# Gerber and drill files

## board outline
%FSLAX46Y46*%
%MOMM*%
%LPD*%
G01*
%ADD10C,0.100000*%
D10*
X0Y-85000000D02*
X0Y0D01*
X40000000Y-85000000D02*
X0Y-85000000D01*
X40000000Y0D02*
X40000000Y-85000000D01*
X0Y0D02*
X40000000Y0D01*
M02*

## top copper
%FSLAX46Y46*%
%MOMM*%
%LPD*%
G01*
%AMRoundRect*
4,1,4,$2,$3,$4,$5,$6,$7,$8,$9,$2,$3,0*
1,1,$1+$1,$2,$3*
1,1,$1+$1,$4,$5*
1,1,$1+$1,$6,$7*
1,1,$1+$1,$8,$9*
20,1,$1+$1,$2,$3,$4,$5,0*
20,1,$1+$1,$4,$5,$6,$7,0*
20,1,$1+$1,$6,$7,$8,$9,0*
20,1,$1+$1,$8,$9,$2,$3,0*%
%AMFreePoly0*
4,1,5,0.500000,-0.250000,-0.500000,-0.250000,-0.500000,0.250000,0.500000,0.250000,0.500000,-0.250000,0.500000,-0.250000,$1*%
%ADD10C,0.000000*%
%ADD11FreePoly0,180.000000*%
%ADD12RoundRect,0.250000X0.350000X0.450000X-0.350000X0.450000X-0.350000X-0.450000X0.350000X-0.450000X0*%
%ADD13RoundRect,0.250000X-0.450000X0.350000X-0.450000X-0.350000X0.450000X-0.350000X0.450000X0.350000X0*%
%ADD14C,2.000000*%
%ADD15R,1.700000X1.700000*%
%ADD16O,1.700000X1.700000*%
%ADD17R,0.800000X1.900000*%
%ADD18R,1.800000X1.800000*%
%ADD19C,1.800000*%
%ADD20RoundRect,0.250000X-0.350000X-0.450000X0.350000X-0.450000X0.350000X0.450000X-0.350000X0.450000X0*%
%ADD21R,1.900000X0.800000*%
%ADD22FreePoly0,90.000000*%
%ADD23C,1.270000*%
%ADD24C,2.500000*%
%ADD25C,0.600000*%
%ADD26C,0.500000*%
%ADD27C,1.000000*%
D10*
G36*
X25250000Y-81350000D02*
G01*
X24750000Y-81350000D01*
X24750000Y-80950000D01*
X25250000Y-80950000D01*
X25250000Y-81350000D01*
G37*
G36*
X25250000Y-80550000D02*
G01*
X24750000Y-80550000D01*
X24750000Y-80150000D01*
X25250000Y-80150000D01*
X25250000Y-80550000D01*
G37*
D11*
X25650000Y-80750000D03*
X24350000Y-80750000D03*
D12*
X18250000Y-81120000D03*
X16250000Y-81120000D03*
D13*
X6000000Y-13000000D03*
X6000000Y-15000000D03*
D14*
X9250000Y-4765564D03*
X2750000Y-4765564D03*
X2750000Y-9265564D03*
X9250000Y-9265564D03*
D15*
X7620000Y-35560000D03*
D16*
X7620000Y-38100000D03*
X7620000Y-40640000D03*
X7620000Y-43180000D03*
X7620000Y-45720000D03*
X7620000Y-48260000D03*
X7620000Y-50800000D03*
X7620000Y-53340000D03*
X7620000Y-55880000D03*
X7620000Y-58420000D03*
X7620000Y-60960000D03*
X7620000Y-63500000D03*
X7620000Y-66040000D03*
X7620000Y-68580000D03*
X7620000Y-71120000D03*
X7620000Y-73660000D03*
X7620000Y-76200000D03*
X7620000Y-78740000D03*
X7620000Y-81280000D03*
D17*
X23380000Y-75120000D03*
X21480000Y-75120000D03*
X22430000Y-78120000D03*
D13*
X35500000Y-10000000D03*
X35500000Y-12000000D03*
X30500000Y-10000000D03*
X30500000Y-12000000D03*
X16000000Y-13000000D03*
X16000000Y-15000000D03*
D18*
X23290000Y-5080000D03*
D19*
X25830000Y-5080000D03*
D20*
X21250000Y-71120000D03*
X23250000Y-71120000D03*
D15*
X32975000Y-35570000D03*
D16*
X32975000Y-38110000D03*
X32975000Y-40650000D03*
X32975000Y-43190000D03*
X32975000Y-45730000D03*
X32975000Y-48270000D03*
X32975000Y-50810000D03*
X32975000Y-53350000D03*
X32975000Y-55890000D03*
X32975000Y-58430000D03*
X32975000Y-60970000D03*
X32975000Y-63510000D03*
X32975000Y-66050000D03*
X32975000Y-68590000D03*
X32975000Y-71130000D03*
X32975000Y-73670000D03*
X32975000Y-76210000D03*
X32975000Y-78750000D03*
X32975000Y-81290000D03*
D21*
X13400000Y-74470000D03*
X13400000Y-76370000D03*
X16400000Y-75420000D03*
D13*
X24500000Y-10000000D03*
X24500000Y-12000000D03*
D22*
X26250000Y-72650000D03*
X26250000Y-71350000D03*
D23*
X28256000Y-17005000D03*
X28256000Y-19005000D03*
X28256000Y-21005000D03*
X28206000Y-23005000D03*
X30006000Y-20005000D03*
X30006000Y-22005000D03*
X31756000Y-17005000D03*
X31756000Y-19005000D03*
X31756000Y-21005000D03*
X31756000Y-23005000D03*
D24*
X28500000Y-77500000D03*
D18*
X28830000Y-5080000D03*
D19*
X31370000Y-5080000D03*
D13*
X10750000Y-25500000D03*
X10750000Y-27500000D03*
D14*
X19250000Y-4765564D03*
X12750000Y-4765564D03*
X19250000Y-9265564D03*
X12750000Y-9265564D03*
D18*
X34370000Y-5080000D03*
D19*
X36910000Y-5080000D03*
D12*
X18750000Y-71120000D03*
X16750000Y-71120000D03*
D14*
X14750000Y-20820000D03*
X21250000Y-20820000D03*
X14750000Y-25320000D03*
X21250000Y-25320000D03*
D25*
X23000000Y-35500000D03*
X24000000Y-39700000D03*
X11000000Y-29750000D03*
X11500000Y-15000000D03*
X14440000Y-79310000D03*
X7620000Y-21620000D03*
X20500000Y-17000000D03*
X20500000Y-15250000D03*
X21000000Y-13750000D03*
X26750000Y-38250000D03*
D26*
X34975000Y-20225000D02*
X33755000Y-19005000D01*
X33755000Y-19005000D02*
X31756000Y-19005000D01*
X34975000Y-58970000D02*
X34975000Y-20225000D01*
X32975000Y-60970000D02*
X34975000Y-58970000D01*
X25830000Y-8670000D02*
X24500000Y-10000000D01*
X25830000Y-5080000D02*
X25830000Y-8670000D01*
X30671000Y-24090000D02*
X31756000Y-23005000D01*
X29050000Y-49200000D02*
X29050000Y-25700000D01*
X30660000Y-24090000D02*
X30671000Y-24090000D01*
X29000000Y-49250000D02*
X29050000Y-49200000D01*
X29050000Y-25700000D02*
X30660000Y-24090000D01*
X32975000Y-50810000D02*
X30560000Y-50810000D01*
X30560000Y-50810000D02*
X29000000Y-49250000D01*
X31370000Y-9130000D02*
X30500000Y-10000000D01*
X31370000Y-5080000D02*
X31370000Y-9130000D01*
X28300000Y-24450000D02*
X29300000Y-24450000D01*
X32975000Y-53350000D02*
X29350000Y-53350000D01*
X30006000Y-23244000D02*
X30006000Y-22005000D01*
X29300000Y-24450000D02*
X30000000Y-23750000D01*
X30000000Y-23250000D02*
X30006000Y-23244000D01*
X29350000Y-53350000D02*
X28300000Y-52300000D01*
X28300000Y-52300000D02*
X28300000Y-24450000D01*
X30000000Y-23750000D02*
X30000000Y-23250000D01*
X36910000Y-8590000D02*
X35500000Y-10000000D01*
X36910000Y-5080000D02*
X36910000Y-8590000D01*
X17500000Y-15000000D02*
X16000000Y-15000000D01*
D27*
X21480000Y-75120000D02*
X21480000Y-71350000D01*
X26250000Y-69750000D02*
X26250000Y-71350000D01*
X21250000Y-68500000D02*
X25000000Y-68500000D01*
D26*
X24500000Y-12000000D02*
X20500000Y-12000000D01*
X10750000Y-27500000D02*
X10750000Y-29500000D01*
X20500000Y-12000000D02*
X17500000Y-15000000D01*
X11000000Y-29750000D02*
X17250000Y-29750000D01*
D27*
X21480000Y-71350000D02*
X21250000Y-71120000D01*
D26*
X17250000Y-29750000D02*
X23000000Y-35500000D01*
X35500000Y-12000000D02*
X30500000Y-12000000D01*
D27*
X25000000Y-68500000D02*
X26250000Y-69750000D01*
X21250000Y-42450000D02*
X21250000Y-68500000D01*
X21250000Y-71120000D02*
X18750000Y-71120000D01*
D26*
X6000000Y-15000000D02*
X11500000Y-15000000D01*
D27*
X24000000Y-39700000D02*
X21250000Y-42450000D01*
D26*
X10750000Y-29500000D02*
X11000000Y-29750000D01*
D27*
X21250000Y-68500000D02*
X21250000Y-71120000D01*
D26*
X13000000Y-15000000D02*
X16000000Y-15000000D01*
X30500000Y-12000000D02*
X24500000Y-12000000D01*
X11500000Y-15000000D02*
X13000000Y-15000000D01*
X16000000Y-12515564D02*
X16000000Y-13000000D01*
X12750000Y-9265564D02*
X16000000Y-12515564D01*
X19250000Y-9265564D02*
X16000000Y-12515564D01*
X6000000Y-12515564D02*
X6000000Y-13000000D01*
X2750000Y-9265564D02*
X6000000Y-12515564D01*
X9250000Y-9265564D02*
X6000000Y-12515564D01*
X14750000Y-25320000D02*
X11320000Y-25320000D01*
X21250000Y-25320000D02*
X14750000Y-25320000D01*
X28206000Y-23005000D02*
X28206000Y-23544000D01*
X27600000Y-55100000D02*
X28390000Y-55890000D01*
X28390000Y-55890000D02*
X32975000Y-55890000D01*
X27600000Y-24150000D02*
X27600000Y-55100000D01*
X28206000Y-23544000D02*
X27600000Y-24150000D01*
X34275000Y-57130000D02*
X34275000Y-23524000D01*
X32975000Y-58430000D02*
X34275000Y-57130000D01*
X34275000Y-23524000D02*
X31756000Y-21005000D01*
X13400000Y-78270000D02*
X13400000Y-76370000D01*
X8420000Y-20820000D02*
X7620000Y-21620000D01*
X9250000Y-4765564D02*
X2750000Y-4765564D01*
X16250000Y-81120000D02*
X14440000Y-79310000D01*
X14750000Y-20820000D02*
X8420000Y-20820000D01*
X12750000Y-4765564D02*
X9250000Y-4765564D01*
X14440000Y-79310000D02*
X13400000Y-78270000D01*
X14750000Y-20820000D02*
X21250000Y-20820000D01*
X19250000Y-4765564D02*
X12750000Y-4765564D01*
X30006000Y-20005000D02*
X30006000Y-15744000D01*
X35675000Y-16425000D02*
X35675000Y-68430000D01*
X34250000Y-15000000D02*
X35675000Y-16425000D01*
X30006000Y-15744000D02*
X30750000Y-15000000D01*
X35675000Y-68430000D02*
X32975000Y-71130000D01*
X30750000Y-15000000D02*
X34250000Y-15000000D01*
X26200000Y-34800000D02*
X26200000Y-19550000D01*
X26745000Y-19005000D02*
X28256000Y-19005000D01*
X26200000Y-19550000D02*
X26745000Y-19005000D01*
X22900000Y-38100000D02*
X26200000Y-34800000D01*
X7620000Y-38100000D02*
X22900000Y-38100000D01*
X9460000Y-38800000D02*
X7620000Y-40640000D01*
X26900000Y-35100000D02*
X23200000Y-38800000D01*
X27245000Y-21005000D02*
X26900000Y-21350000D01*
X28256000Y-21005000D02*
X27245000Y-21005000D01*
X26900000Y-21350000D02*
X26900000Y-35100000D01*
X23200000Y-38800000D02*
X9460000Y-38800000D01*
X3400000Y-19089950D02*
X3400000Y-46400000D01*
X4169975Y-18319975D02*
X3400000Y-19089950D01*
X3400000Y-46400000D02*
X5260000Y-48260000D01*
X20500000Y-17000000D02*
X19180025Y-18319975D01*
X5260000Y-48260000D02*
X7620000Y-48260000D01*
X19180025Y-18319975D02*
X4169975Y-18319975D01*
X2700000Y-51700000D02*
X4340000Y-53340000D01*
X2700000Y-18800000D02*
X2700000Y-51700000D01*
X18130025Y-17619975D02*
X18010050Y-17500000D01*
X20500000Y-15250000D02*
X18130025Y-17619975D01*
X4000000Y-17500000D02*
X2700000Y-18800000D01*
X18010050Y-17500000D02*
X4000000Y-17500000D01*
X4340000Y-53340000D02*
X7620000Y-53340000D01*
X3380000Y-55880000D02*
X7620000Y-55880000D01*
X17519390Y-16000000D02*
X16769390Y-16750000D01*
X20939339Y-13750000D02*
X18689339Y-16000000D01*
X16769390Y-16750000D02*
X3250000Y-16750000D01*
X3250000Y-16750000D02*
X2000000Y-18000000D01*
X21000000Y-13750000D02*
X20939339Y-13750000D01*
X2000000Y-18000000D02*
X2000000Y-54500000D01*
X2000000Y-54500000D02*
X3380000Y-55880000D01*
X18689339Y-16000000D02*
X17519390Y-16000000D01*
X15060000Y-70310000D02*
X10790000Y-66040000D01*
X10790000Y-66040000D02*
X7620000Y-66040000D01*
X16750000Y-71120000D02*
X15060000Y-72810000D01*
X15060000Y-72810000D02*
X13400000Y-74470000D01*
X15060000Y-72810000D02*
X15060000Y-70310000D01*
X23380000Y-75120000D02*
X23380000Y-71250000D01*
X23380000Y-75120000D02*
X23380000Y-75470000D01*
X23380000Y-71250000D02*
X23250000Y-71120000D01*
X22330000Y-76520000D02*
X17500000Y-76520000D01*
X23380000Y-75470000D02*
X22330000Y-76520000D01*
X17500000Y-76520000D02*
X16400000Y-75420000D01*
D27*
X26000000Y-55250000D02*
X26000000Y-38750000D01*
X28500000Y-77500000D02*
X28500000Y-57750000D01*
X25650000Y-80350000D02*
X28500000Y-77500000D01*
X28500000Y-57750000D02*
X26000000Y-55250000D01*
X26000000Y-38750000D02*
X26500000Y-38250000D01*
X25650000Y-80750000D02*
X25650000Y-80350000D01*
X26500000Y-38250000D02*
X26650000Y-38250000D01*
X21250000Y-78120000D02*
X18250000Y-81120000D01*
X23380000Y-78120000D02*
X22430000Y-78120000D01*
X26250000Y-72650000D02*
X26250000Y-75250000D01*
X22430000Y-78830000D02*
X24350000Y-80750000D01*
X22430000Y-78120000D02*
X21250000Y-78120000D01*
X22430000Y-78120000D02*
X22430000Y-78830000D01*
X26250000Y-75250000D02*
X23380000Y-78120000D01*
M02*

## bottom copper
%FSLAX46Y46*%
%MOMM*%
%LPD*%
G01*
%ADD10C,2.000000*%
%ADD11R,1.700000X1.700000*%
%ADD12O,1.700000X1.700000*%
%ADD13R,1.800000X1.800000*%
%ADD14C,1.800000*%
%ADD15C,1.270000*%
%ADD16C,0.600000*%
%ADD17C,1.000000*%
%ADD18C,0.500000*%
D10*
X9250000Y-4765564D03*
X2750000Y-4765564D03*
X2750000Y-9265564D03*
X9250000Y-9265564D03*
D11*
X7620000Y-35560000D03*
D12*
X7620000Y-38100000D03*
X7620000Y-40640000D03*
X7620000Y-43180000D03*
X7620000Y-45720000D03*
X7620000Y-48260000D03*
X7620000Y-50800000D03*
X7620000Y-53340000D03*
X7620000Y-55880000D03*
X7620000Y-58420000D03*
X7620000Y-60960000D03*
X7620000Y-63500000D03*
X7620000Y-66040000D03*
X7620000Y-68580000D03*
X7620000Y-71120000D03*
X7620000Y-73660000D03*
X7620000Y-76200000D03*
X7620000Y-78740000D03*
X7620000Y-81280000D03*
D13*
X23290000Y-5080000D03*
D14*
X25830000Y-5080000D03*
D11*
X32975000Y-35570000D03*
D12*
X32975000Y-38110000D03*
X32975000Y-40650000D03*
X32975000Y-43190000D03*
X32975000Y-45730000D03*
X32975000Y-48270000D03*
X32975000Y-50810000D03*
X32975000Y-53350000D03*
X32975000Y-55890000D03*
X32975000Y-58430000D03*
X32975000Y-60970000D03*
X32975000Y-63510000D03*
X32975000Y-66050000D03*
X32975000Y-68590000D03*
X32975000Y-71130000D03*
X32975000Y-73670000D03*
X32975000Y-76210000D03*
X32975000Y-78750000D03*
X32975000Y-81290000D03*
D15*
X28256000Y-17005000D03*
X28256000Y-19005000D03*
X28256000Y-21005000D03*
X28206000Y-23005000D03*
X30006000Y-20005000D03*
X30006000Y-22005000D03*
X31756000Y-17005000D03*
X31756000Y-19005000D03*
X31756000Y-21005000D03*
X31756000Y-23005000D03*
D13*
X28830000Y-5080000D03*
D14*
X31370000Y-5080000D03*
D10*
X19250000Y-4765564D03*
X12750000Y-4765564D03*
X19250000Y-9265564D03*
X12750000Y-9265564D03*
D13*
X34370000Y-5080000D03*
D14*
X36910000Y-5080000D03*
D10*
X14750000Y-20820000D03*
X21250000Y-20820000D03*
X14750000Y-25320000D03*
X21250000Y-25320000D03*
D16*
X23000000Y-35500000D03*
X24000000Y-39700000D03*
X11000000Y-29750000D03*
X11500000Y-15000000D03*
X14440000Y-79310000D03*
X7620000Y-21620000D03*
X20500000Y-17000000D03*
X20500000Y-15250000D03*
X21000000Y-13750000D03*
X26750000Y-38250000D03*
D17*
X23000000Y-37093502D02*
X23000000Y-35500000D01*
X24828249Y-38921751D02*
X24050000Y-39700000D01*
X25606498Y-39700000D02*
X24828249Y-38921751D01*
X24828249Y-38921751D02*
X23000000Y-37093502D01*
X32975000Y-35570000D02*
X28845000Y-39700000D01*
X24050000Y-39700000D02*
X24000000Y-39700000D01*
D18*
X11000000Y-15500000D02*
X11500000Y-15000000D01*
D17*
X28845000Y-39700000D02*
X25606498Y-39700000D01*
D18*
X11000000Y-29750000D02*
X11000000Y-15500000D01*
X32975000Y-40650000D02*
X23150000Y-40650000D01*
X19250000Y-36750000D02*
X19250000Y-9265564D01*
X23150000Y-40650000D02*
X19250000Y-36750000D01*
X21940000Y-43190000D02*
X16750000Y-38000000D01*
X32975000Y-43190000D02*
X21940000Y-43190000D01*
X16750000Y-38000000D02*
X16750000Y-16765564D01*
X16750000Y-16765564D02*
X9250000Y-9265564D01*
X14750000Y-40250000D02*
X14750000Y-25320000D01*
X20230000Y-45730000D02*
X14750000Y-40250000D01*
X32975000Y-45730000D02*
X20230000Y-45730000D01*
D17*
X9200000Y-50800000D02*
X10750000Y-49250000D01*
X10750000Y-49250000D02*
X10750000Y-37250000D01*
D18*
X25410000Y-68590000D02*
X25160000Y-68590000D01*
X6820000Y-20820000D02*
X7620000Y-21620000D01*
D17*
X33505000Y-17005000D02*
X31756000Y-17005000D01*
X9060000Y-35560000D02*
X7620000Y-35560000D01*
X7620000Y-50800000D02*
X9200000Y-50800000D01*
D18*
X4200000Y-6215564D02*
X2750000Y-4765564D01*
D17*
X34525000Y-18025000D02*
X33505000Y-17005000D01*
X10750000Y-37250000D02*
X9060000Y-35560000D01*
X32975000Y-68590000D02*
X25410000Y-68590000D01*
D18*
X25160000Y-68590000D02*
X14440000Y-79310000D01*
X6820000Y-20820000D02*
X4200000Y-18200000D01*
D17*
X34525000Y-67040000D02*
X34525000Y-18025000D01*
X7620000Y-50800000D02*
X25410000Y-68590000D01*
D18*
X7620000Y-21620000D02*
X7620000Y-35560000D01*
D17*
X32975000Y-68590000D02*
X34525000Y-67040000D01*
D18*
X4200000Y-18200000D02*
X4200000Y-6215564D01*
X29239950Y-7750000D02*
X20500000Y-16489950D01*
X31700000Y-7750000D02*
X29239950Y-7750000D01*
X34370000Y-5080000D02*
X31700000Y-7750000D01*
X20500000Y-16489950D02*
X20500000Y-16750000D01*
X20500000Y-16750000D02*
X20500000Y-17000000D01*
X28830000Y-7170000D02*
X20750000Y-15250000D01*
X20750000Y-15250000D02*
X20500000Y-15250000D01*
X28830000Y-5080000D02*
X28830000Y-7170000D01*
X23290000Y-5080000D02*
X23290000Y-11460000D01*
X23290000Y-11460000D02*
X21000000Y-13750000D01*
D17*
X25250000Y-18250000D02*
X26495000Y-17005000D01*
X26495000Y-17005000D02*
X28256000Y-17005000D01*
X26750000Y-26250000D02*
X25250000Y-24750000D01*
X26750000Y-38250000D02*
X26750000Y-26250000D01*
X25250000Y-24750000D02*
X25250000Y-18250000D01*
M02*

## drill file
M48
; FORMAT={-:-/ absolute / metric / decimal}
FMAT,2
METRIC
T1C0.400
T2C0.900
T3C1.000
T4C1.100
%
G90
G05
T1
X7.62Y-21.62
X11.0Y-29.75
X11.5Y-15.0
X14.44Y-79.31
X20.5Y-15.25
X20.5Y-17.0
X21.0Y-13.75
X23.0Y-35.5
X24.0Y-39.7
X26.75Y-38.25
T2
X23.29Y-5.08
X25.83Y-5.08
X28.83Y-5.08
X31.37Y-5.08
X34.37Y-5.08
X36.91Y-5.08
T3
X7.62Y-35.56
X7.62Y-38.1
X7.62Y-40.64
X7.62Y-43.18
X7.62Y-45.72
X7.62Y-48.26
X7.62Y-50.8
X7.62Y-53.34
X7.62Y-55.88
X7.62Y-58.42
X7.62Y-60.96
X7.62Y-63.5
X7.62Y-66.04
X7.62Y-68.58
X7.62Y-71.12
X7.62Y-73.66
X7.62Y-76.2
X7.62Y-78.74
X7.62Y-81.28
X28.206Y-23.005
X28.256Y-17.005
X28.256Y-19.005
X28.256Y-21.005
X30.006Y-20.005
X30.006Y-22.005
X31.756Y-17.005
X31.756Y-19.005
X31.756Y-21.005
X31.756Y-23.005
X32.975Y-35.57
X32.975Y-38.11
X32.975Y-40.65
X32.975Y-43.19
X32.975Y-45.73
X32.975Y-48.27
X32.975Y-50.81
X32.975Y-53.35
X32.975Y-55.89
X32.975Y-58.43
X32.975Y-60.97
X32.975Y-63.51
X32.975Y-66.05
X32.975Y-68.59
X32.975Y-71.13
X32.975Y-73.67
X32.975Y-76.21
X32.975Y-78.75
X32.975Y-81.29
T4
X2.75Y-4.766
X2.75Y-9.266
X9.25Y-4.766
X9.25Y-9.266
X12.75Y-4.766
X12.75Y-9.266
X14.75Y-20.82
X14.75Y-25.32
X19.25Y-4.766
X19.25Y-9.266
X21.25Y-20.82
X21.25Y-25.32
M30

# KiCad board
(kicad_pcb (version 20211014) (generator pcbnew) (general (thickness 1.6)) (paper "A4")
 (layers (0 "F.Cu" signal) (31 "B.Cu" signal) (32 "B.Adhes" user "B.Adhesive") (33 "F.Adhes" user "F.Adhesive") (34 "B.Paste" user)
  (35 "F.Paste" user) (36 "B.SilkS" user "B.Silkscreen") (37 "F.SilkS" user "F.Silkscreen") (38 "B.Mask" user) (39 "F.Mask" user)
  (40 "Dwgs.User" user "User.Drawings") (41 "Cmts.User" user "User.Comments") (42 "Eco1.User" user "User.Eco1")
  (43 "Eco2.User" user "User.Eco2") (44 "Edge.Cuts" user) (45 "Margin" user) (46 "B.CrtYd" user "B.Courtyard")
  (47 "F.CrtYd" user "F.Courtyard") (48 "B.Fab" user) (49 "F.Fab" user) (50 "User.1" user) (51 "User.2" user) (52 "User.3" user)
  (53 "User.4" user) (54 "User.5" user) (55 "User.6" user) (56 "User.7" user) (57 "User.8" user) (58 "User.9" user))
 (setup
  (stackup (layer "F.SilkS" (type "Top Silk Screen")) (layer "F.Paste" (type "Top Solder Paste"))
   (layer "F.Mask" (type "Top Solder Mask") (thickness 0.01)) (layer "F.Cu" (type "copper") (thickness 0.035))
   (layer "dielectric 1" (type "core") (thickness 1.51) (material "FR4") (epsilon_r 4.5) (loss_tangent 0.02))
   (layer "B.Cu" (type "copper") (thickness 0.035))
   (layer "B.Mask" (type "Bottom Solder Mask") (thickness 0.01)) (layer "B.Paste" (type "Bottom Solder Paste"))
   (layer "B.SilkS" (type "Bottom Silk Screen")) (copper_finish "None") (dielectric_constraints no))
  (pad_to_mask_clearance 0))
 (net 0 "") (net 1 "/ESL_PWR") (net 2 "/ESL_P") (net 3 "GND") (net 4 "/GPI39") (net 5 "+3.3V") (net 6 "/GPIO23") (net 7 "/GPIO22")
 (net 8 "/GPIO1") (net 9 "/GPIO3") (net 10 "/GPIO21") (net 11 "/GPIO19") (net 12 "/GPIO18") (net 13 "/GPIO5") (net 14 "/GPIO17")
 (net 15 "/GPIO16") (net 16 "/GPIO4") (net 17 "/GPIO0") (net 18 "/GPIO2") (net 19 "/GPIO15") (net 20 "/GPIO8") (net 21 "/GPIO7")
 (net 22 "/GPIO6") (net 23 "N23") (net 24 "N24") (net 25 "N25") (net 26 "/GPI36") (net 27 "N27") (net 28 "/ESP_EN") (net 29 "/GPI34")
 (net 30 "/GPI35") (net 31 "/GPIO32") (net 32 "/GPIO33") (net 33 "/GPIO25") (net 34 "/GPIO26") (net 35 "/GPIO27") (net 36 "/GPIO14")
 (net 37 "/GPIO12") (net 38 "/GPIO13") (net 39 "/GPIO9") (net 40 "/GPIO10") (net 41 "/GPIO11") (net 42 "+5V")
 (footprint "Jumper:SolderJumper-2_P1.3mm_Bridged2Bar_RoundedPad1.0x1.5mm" (layer "F.Cu") (at 25 80.75 180)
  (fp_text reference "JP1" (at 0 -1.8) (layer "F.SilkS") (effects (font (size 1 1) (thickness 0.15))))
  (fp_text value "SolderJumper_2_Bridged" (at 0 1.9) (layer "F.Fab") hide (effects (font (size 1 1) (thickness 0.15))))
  (fp_poly (pts (xy -0.25 -0.6) (xy 0.25 -0.6) (xy 0.25 -0.2) (xy -0.25 -0.2)) (layer "F.Cu") (width 0) (fill solid))
  (fp_poly (pts (xy -0.25 0.2) (xy 0.25 0.2) (xy 0.25 0.6) (xy -0.25 0.6)) (layer "F.Cu") (width 0) (fill solid))
  (pad "1" smd custom (at -0.65 0 180) (size 1 0.5) (layers "F.Cu" "F.Mask") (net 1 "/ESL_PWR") (zone_connect 2)
   (options (clearance outline) (anchor rect)) (primitives))
  (pad "2" smd custom (at 0.65 0 180) (size 1 0.5) (layers "F.Cu" "F.Mask") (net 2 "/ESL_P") (zone_connect 2)
   (options (clearance outline) (anchor rect)) (primitives)))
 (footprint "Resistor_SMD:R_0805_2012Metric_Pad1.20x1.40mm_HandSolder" (layer "F.Cu") (at 17.25 81.12 180)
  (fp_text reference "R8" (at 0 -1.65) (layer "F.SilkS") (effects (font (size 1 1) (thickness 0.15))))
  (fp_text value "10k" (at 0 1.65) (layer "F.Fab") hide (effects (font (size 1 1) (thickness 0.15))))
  (pad "1" smd roundrect (at -1 0 180) (size 1.2 1.4) (layers "F.Cu" "F.Paste" "F.Mask") (roundrect_rratio 0.2083333333) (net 2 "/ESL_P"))
  (pad "2" smd roundrect (at 1 0 180) (size 1.2 1.4) (layers "F.Cu" "F.Paste" "F.Mask") (roundrect_rratio 0.2083333333) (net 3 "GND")))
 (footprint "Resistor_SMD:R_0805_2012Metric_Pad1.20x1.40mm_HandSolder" (layer "F.Cu") (at 6 14 -90)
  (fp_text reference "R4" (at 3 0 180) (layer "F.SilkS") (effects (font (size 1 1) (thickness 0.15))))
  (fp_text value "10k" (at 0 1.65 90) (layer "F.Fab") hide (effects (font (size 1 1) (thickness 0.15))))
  (pad "1" smd roundrect (at -1 0 270) (size 1.2 1.4) (layers "F.Cu" "F.Paste" "F.Mask") (roundrect_rratio 0.2083333333) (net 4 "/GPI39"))
  (pad "2" smd roundrect (at 1 0 270) (size 1.2 1.4) (layers "F.Cu" "F.Paste" "F.Mask") (roundrect_rratio 0.2083333333) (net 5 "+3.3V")))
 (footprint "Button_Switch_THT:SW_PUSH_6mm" (layer "F.Cu") (at 2.75 4.765564)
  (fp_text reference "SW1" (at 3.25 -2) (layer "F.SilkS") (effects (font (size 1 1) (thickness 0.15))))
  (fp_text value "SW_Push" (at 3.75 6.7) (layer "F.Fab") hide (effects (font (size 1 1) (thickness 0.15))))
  (pad "1" thru_hole circle (at 6.5 0 90) (size 2 2) (drill 1.1) (layers *.Cu *.Mask) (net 3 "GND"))
  (pad "1" thru_hole circle (at 0 0 90) (size 2 2) (drill 1.1) (layers *.Cu *.Mask) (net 3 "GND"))
  (pad "2" thru_hole circle (at 0 4.5 90) (size 2 2) (drill 1.1) (layers *.Cu *.Mask) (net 4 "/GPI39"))
  (pad "2" thru_hole circle (at 6.5 4.5 90) (size 2 2) (drill 1.1) (layers *.Cu *.Mask) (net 4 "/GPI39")))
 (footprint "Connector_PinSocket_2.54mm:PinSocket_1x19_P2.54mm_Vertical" (layer "F.Cu") (at 7.62 35.56)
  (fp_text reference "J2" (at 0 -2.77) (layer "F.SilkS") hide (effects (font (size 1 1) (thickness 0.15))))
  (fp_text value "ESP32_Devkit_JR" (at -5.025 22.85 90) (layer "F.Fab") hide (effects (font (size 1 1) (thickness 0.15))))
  (pad "1" thru_hole rect (at 0 0) (size 1.7 1.7) (drill 1) (layers *.Cu *.Mask) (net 3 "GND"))
  (pad "2" thru_hole oval (at 0 2.54) (size 1.7 1.7) (drill 1) (layers *.Cu *.Mask) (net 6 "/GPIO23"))
  (pad "3" thru_hole oval (at 0 5.08) (size 1.7 1.7) (drill 1) (layers *.Cu *.Mask) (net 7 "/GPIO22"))
  (pad "4" thru_hole oval (at 0 7.62) (size 1.7 1.7) (drill 1) (layers *.Cu *.Mask) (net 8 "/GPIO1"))
  (pad "5" thru_hole oval (at 0 10.16) (size 1.7 1.7) (drill 1) (layers *.Cu *.Mask) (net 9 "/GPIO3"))
  (pad "6" thru_hole oval (at 0 12.7) (size 1.7 1.7) (drill 1) (layers *.Cu *.Mask) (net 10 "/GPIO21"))
  (pad "7" thru_hole oval (at 0 15.24) (size 1.7 1.7) (drill 1) (layers *.Cu *.Mask) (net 3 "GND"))
  (pad "8" thru_hole oval (at 0 17.78) (size 1.7 1.7) (drill 1) (layers *.Cu *.Mask) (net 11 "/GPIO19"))
  (pad "9" thru_hole oval (at 0 20.32) (size 1.7 1.7) (drill 1) (layers *.Cu *.Mask) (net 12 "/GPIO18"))
  (pad "10" thru_hole oval (at 0 22.86) (size 1.7 1.7) (drill 1) (layers *.Cu *.Mask) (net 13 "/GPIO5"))
  (pad "11" thru_hole oval (at 0 25.4) (size 1.7 1.7) (drill 1) (layers *.Cu *.Mask) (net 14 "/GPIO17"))
  (pad "12" thru_hole oval (at 0 27.94) (size 1.7 1.7) (drill 1) (layers *.Cu *.Mask) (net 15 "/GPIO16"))
  (pad "13" thru_hole oval (at 0 30.48) (size 1.7 1.7) (drill 1) (layers *.Cu *.Mask) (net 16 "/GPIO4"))
  (pad "14" thru_hole oval (at 0 33.02) (size 1.7 1.7) (drill 1) (layers *.Cu *.Mask) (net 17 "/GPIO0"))
  (pad "15" thru_hole oval (at 0 35.56) (size 1.7 1.7) (drill 1) (layers *.Cu *.Mask) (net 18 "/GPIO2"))
  (pad "16" thru_hole oval (at 0 38.1) (size 1.7 1.7) (drill 1) (layers *.Cu *.Mask) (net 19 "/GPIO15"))
  (pad "17" thru_hole oval (at 0 40.64) (size 1.7 1.7) (drill 1) (layers *.Cu *.Mask) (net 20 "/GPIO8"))
  (pad "18" thru_hole oval (at 0 43.18) (size 1.7 1.7) (drill 1) (layers *.Cu *.Mask) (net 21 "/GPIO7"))
  (pad "19" thru_hole oval (at 0 45.72) (size 1.7 1.7) (drill 1) (layers *.Cu *.Mask) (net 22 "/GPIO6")))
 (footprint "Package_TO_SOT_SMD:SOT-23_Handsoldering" (layer "F.Cu") (at 22.43 76.62 -90)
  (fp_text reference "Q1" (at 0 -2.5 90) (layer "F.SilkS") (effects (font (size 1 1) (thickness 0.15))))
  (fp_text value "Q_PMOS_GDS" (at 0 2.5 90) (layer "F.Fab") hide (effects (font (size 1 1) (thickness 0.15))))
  (pad "1" smd rect (at -1.5 -0.95 270) (size 1.9 0.8) (layers "F.Cu" "F.Paste" "F.Mask") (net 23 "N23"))
  (pad "2" smd rect (at -1.5 0.95 270) (size 1.9 0.8) (layers "F.Cu" "F.Paste" "F.Mask") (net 5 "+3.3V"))
  (pad "3" smd rect (at 1.5 0 270) (size 1.9 0.8) (layers "F.Cu" "F.Paste" "F.Mask") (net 2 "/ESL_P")))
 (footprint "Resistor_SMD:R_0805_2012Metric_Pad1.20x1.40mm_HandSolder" (layer "F.Cu") (at 35.5 11 -90)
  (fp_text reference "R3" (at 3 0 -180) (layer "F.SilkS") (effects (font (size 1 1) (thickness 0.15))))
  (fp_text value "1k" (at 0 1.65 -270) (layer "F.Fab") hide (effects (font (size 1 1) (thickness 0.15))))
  (pad "1" smd roundrect (at -1 0 270) (size 1.2 1.4) (layers "F.Cu" "F.Paste" "F.Mask") (roundrect_rratio 0.2083333333) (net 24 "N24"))
  (pad "2" smd roundrect (at 1 0 270) (size 1.2 1.4) (layers "F.Cu" "F.Paste" "F.Mask") (roundrect_rratio 0.2083333333) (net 5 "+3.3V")))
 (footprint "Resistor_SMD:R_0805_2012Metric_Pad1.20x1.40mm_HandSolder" (layer "F.Cu") (at 30.5 11 -90)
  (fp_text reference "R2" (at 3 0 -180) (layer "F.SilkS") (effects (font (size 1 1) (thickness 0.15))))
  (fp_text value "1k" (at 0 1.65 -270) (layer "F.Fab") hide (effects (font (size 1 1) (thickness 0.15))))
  (pad "1" smd roundrect (at -1 0 270) (size 1.2 1.4) (layers "F.Cu" "F.Paste" "F.Mask") (roundrect_rratio 0.2083333333) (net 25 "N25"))
  (pad "2" smd roundrect (at 1 0 270) (size 1.2 1.4) (layers "F.Cu" "F.Paste" "F.Mask") (roundrect_rratio 0.2083333333) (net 5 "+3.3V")))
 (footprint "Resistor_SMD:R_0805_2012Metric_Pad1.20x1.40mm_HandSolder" (layer "F.Cu") (at 16 14 -90)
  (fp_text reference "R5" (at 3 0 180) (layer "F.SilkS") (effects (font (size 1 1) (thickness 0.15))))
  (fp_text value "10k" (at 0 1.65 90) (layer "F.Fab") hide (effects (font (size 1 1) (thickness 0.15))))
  (pad "1" smd roundrect (at -1 0 270) (size 1.2 1.4) (layers "F.Cu" "F.Paste" "F.Mask") (roundrect_rratio 0.2083333333) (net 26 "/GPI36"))
  (pad "2" smd roundrect (at 1 0 270) (size 1.2 1.4) (layers "F.Cu" "F.Paste" "F.Mask") (roundrect_rratio 0.2083333333) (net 5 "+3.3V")))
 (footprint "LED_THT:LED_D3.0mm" (layer "F.Cu") (at 23.29 5.08)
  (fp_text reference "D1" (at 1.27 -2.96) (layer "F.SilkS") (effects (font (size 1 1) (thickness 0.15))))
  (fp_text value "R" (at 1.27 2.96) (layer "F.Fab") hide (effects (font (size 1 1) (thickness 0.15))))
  (pad "1" thru_hole rect (at 0 0) (size 1.8 1.8) (drill 0.9) (layers *.Cu *.Mask) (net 12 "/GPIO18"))
  (pad "2" thru_hole circle (at 2.54 0) (size 1.8 1.8) (drill 0.9) (layers *.Cu *.Mask) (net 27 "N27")))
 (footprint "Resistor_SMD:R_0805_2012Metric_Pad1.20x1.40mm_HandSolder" (layer "F.Cu") (at 22.25 71.12)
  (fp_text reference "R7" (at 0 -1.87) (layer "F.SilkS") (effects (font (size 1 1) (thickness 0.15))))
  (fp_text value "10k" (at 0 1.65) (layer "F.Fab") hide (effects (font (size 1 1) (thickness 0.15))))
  (pad "1" smd roundrect (at -1 0) (size 1.2 1.4) (layers "F.Cu" "F.Paste" "F.Mask") (roundrect_rratio 0.2083333333) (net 5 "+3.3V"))
  (pad "2" smd roundrect (at 1 0) (size 1.2 1.4) (layers "F.Cu" "F.Paste" "F.Mask") (roundrect_rratio 0.2083333333) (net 23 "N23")))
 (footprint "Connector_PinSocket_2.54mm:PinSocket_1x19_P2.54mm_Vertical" (layer "F.Cu") (at 32.975 35.57)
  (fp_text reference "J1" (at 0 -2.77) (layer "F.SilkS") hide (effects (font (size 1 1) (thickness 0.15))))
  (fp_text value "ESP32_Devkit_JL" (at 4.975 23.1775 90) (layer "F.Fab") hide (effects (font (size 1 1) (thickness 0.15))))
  (pad "1" thru_hole rect (at 0 0) (size 1.7 1.7) (drill 1) (layers *.Cu *.Mask) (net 5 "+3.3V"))
  (pad "2" thru_hole oval (at 0 2.54) (size 1.7 1.7) (drill 1) (layers *.Cu *.Mask) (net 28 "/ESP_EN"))
  (pad "3" thru_hole oval (at 0 5.08) (size 1.7 1.7) (drill 1) (layers *.Cu *.Mask) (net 26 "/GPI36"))
  (pad "4" thru_hole oval (at 0 7.62) (size 1.7 1.7) (drill 1) (layers *.Cu *.Mask) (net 4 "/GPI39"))
  (pad "5" thru_hole oval (at 0 10.16) (size 1.7 1.7) (drill 1) (layers *.Cu *.Mask) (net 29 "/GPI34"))
  (pad "6" thru_hole oval (at 0 12.7) (size 1.7 1.7) (drill 1) (layers *.Cu *.Mask) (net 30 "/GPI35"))
  (pad "7" thru_hole oval (at 0 15.24) (size 1.7 1.7) (drill 1) (layers *.Cu *.Mask) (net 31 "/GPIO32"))
  (pad "8" thru_hole oval (at 0 17.78) (size 1.7 1.7) (drill 1) (layers *.Cu *.Mask) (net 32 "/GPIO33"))
  (pad "9" thru_hole oval (at 0 20.32) (size 1.7 1.7) (drill 1) (layers *.Cu *.Mask) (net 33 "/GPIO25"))
  (pad "10" thru_hole oval (at 0 22.86) (size 1.7 1.7) (drill 1) (layers *.Cu *.Mask) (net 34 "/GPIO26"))
  (pad "11" thru_hole oval (at 0 25.4) (size 1.7 1.7) (drill 1) (layers *.Cu *.Mask) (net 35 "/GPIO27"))
  (pad "12" thru_hole oval (at 0 27.94) (size 1.7 1.7) (drill 1) (layers *.Cu *.Mask) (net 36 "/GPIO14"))
  (pad "13" thru_hole oval (at 0 30.48) (size 1.7 1.7) (drill 1) (layers *.Cu *.Mask) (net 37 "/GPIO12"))
  (pad "14" thru_hole oval (at 0 33.02) (size 1.7 1.7) (drill 1) (layers *.Cu *.Mask) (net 3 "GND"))
  (pad "15" thru_hole oval (at 0 35.56) (size 1.7 1.7) (drill 1) (layers *.Cu *.Mask) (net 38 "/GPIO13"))
  (pad "16" thru_hole oval (at 0 38.1) (size 1.7 1.7) (drill 1) (layers *.Cu *.Mask) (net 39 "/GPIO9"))
  (pad "17" thru_hole oval (at 0 40.64) (size 1.7 1.7) (drill 1) (layers *.Cu *.Mask) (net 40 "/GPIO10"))
  (pad "18" thru_hole oval (at 0 43.18) (size 1.7 1.7) (drill 1) (layers *.Cu *.Mask) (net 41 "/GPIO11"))
  (pad "19" thru_hole oval (at 0 45.72) (size 1.7 1.7) (drill 1) (layers *.Cu *.Mask) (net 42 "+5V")))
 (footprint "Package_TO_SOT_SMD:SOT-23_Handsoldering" (layer "F.Cu") (at 14.9 75.42)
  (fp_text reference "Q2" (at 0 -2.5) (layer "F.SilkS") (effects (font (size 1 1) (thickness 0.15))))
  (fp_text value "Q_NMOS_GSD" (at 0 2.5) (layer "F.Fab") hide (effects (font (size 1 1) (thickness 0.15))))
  (pad "1" smd rect (at -1.5 -0.95) (size 1.9 0.8) (layers "F.Cu" "F.Paste" "F.Mask") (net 16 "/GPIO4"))
  (pad "2" smd rect (at -1.5 0.95) (size 1.9 0.8) (layers "F.Cu" "F.Paste" "F.Mask") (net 3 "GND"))
  (pad "3" smd rect (at 1.5 0) (size 1.9 0.8) (layers "F.Cu" "F.Paste" "F.Mask") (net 23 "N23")))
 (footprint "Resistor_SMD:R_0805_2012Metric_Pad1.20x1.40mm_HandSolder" (layer "F.Cu") (at 24.5 11 -90)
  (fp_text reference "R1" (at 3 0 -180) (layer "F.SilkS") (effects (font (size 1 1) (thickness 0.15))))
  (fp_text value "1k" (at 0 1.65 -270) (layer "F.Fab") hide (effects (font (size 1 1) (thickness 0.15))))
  (pad "1" smd roundrect (at -1 0 270) (size 1.2 1.4) (layers "F.Cu" "F.Paste" "F.Mask") (roundrect_rratio 0.2083333333) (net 27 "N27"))
  (pad "2" smd roundrect (at 1 0 270) (size 1.2 1.4) (layers "F.Cu" "F.Paste" "F.Mask") (roundrect_rratio 0.2083333333) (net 5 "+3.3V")))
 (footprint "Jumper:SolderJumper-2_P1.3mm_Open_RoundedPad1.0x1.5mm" (layer "F.Cu") (at 26.25 72 90)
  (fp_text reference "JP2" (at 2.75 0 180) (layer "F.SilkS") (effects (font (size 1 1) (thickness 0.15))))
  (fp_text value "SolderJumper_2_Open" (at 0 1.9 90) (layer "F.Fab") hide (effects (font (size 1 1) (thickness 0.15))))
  (pad "1" smd custom (at -0.65 0 90) (size 1 0.5) (layers "F.Cu" "F.Mask") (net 2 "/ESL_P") (zone_connect 2)
   (options (clearance outline) (anchor rect)) (primitives))
  (pad "2" smd custom (at 0.65 0 90) (size 1 0.5) (layers "F.Cu" "F.Mask") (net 5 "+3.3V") (zone_connect 2)
   (options (clearance outline) (anchor rect)) (primitives)))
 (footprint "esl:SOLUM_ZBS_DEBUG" (layer "F.Cu") (at 30 20 -90)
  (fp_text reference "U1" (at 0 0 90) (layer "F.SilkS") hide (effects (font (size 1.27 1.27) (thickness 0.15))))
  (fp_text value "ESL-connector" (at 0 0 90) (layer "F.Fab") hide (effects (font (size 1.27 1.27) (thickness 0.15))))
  (pad "1" thru_hole circle (at -2.995 1.744 270) (size 1.27 1.27) (drill 1) (layers *.Cu *.Mask) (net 1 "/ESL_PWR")
   (solder_mask_margin 0.0508))
  (pad "2" thru_hole circle (at -0.995 1.744 270) (size 1.27 1.27) (drill 1) (layers *.Cu *.Mask) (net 6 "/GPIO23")
   (solder_mask_margin 0.0508))
  (pad "3" thru_hole circle (at 1.005 1.744 270) (size 1.27 1.27) (drill 1) (layers *.Cu *.Mask) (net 7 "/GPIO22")
   (solder_mask_margin 0.0508))
  (pad "4" thru_hole circle (at 3.005 1.794 270) (size 1.27 1.27) (drill 1) (layers *.Cu *.Mask) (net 33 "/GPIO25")
   (solder_mask_margin 0.0508))
  (pad "5" thru_hole circle (at 0.005 -0.006 270) (size 1.27 1.27) (drill 1) (layers *.Cu *.Mask) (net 38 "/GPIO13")
   (solder_mask_margin 0.0508))
  (pad "6" thru_hole circle (at 2.005 -0.006 270) (size 1.27 1.27) (drill 1) (layers *.Cu *.Mask) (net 32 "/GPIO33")
   (solder_mask_margin 0.0508))
  (pad "7" thru_hole circle (at -2.995 -1.756 270) (size 1.27 1.27) (drill 1) (layers *.Cu *.Mask) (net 3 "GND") (solder_mask_margin 0.0508))
  (pad "8" thru_hole circle (at -0.995 -1.756 270) (size 1.27 1.27) (drill 1) (layers *.Cu *.Mask) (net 35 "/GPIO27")
   (solder_mask_margin 0.0508))
  (pad "9" thru_hole circle (at 1.005 -1.756 270) (size 1.27 1.27) (drill 1) (layers *.Cu *.Mask) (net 34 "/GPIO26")
   (solder_mask_margin 0.0508))
  (pad "10" thru_hole circle (at 3.005 -1.756 270) (size 1.27 1.27) (drill 1) (layers *.Cu *.Mask) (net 31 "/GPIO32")
   (solder_mask_margin 0.0508)))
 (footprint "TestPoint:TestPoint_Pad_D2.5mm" (layer "F.Cu") (at 28.5 77.5)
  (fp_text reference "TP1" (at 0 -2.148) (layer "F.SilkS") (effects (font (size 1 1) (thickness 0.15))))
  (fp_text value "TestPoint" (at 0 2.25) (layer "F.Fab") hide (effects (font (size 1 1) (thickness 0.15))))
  (pad "1" smd circle (at 0 0) (size 2.5 2.5) (layers "F.Cu" "F.Mask") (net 1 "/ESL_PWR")))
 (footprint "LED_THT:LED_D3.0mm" (layer "F.Cu") (at 28.83 5.08)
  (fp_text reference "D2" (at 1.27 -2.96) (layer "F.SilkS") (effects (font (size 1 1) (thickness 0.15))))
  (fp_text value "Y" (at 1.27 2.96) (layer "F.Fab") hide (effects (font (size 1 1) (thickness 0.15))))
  (pad "1" thru_hole rect (at 0 0) (size 1.8 1.8) (drill 0.9) (layers *.Cu *.Mask) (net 11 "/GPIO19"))
  (pad "2" thru_hole circle (at 2.54 0) (size 1.8 1.8) (drill 0.9) (layers *.Cu *.Mask) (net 25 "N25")))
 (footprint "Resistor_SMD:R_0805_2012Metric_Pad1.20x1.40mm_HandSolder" (layer "F.Cu") (at 10.75 26.5 -90)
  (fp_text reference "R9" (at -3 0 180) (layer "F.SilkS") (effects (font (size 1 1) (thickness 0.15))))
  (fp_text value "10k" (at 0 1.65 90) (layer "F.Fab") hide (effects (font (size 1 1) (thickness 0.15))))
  (pad "1" smd roundrect (at -1 0 270) (size 1.2 1.4) (layers "F.Cu" "F.Paste" "F.Mask") (roundrect_rratio 0.2083333333) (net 29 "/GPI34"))
  (pad "2" smd roundrect (at 1 0 270) (size 1.2 1.4) (layers "F.Cu" "F.Paste" "F.Mask") (roundrect_rratio 0.2083333333) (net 5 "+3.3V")))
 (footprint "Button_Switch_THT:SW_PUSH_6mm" (layer "F.Cu") (at 12.75 4.765564)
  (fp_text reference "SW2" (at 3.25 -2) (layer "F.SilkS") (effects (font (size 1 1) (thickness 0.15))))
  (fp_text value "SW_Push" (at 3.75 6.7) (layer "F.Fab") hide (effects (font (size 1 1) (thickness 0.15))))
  (pad "1" thru_hole circle (at 6.5 0 90) (size 2 2) (drill 1.1) (layers *.Cu *.Mask) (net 3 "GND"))
  (pad "1" thru_hole circle (at 0 0 90) (size 2 2) (drill 1.1) (layers *.Cu *.Mask) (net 3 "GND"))
  (pad "2" thru_hole circle (at 6.5 4.5 90) (size 2 2) (drill 1.1) (layers *.Cu *.Mask) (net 26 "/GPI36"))
  (pad "2" thru_hole circle (at 0 4.5 90) (size 2 2) (drill 1.1) (layers *.Cu *.Mask) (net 26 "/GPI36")))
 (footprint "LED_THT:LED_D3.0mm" (layer "F.Cu") (at 34.37 5.08)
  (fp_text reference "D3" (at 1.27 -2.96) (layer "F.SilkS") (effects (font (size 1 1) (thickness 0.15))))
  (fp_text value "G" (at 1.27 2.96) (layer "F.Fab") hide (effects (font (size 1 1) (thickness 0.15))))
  (pad "1" thru_hole rect (at 0 0) (size 1.8 1.8) (drill 0.9) (layers *.Cu *.Mask) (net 10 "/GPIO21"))
  (pad "2" thru_hole circle (at 2.54 0) (size 1.8 1.8) (drill 0.9) (layers *.Cu *.Mask) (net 24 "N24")))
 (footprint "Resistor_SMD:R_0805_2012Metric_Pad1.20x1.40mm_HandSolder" (layer "F.Cu") (at 17.75 71.12 180)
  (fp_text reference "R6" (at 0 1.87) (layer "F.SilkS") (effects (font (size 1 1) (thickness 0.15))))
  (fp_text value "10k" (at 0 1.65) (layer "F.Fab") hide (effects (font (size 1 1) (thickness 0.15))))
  (pad "1" smd roundrect (at -1 0 180) (size 1.2 1.4) (layers "F.Cu" "F.Paste" "F.Mask") (roundrect_rratio 0.2083333333) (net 5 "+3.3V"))
  (pad "2" smd roundrect (at 1 0 180) (size 1.2 1.4) (layers "F.Cu" "F.Paste" "F.Mask") (roundrect_rratio 0.2083333333) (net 16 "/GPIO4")))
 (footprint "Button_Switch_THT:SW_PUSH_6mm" (layer "B.Cu") (at 21.25 20.82 180)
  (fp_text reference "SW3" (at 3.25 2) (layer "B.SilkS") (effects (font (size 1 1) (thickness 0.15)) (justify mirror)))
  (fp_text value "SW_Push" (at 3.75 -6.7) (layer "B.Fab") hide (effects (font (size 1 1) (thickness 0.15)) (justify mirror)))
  (pad "1" thru_hole circle locked (at 6.5 0 90) (size 2 2) (drill 1.1) (layers *.Cu *.Mask) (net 3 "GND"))
  (pad "1" thru_hole circle (at 0 0 90) (size 2 2) (drill 1.1) (layers *.Cu *.Mask) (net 3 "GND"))
  (pad "2" thru_hole circle (at 6.5 -4.5 90) (size 2 2) (drill 1.1) (layers *.Cu *.Mask) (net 29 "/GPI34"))
  (pad "2" thru_hole circle (at 0 -4.5 90) (size 2 2) (drill 1.1) (layers *.Cu *.Mask) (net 29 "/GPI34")))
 (gr_line (start 0 85) (end 0 0) (layer "Edge.Cuts") (width 0.1))
 (gr_line (start 40 85) (end 0 85) (layer "Edge.Cuts") (width 0.1))
 (gr_line (start 40 0) (end 40 85) (layer "Edge.Cuts") (width 0.1))
 (gr_line (start 0 0) (end 40 0) (layer "Edge.Cuts") (width 0.1))
 (segment (start 34.975 20.225) (end 33.755 19.005) (width 0.5) (layer "F.Cu") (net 35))
 (segment (start 33.755 19.005) (end 31.756 19.005) (width 0.5) (layer "F.Cu") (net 35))
 (segment (start 34.975 58.97) (end 34.975 20.225) (width 0.5) (layer "F.Cu") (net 35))
 (segment (start 32.975 60.97) (end 34.975 58.97) (width 0.5) (layer "F.Cu") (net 35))
 (segment (start 25.83 8.67) (end 24.5 10) (width 0.5) (layer "F.Cu") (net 27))
 (segment (start 25.83 5.08) (end 25.83 8.67) (width 0.5) (layer "F.Cu") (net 27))
 (segment (start 30.671 24.09) (end 31.756 23.005) (width 0.5) (layer "F.Cu") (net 31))
 (segment (start 29.05 49.2) (end 29.05 25.7) (width 0.5) (layer "F.Cu") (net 31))
 (segment (start 30.66 24.09) (end 30.671 24.09) (width 0.5) (layer "F.Cu") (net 31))
 (segment (start 29 49.25) (end 29.05 49.2) (width 0.5) (layer "F.Cu") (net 31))
 (segment (start 29.05 25.7) (end 30.66 24.09) (width 0.5) (layer "F.Cu") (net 31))
 (segment (start 32.975 50.81) (end 30.56 50.81) (width 0.5) (layer "F.Cu") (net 31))
 (segment (start 30.56 50.81) (end 29 49.25) (width 0.5) (layer "F.Cu") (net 31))
 (segment (start 31.37 9.13) (end 30.5 10) (width 0.5) (layer "F.Cu") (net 25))
 (segment (start 31.37 5.08) (end 31.37 9.13) (width 0.5) (layer "F.Cu") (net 25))
 (segment (start 28.3 24.45) (end 29.3 24.45) (width 0.5) (layer "F.Cu") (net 32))
 (segment (start 32.975 53.35) (end 29.35 53.35) (width 0.5) (layer "F.Cu") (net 32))
 (segment (start 30.006 23.244) (end 30.006 22.005) (width 0.5) (layer "F.Cu") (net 32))
 (segment (start 29.3 24.45) (end 30 23.75) (width 0.5) (layer "F.Cu") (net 32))
 (segment (start 30 23.25) (end 30.006 23.244) (width 0.5) (layer "F.Cu") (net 32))
 (segment (start 29.35 53.35) (end 28.3 52.3) (width 0.5) (layer "F.Cu") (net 32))
 (segment (start 28.3 52.3) (end 28.3 24.45) (width 0.5) (layer "F.Cu") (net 32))
 (segment (start 30 23.75) (end 30 23.25) (width 0.5) (layer "F.Cu") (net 32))
 (segment (start 36.91 8.59) (end 35.5 10) (width 0.5) (layer "F.Cu") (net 24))
 (segment (start 36.91 5.08) (end 36.91 8.59) (width 0.5) (layer "F.Cu") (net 24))
 (segment (start 17.5 15) (end 16 15) (width 0.5) (layer "F.Cu") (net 5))
 (segment (start 21.48 75.12) (end 21.48 71.35) (width 1) (layer "F.Cu") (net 5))
 (segment (start 26.25 69.75) (end 26.25 71.35) (width 1) (layer "F.Cu") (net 5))
 (segment (start 21.25 68.5) (end 25 68.5) (width 1) (layer "F.Cu") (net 5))
 (segment (start 24.5 12) (end 20.5 12) (width 0.5) (layer "F.Cu") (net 5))
 (segment (start 10.75 27.5) (end 10.75 29.5) (width 0.5) (layer "F.Cu") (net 5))
 (segment (start 20.5 12) (end 17.5 15) (width 0.5) (layer "F.Cu") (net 5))
 (segment (start 11 29.75) (end 17.25 29.75) (width 0.5) (layer "F.Cu") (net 5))
 (segment (start 21.48 71.35) (end 21.25 71.12) (width 1) (layer "F.Cu") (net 5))
 (segment (start 17.25 29.75) (end 23 35.5) (width 0.5) (layer "F.Cu") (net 5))
 (segment (start 35.5 12) (end 30.5 12) (width 0.5) (layer "F.Cu") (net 5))
 (segment (start 25 68.5) (end 26.25 69.75) (width 1) (layer "F.Cu") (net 5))
 (segment (start 21.25 42.45) (end 21.25 68.5) (width 1) (layer "F.Cu") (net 5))
 (segment (start 21.25 71.12) (end 18.75 71.12) (width 1) (layer "F.Cu") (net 5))
 (segment (start 6 15) (end 11.5 15) (width 0.5) (layer "F.Cu") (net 5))
 (segment (start 24 39.7) (end 21.25 42.45) (width 1) (layer "F.Cu") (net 5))
 (segment (start 10.75 29.5) (end 11 29.75) (width 0.5) (layer "F.Cu") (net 5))
 (segment (start 21.25 68.5) (end 21.25 71.12) (width 1) (layer "F.Cu") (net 5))
 (segment (start 13 15) (end 16 15) (width 0.5) (layer "F.Cu") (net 5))
 (segment (start 30.5 12) (end 24.5 12) (width 0.5) (layer "F.Cu") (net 5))
 (segment (start 11.5 15) (end 13 15) (width 0.5) (layer "F.Cu") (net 5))
 (via (at 23 35.5) (size 0.6) (drill 0.4) (layers "F.Cu" "B.Cu") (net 5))
 (via (at 24 39.7) (size 0.6) (drill 0.4) (layers "F.Cu" "B.Cu") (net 5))
 (via (at 11 29.75) (size 0.6) (drill 0.4) (layers "F.Cu" "B.Cu") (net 5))
 (via (at 11.5 15) (size 0.6) (drill 0.4) (layers "F.Cu" "B.Cu") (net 5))
 (segment (start 23 37.093502) (end 23 35.5) (width 1) (layer "B.Cu") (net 5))
 (segment (start 24.828249 38.921751) (end 24.05 39.7) (width 1) (layer "B.Cu") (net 5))
 (segment (start 25.606498 39.7) (end 24.828249 38.921751) (width 1) (layer "B.Cu") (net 5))
 (segment (start 24.828249 38.921751) (end 23 37.093502) (width 1) (layer "B.Cu") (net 5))
 (segment (start 32.975 35.57) (end 28.845 39.7) (width 1) (layer "B.Cu") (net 5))
 (segment (start 24.05 39.7) (end 24 39.7) (width 1) (layer "B.Cu") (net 5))
 (segment (start 11 15.5) (end 11.5 15) (width 0.5) (layer "B.Cu") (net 5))
 (segment (start 28.845 39.7) (end 25.606498 39.7) (width 1) (layer "B.Cu") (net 5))
 (segment (start 11 29.75) (end 11 15.5) (width 0.5) (layer "B.Cu") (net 5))
 (segment (start 16 12.515564) (end 16 13) (width 0.5) (layer "F.Cu") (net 26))
 (segment (start 12.75 9.265564) (end 16 12.515564) (width 0.5) (layer "F.Cu") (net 26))
 (segment (start 19.25 9.265564) (end 16 12.515564) (width 0.5) (layer "F.Cu") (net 26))
 (segment (start 32.975 40.65) (end 23.15 40.65) (width 0.5) (layer "B.Cu") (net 26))
 (segment (start 19.25 36.75) (end 19.25 9.265564) (width 0.5) (layer "B.Cu") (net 26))
 (segment (start 23.15 40.65) (end 19.25 36.75) (width 0.5) (layer "B.Cu") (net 26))
 (segment (start 6 12.515564) (end 6 13) (width 0.5) (layer "F.Cu") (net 4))
 (segment (start 2.75 9.265564) (end 6 12.515564) (width 0.5) (layer "F.Cu") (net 4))
 (segment (start 9.25 9.265564) (end 6 12.515564) (width 0.5) (layer "F.Cu") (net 4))
 (segment (start 21.94 43.19) (end 16.75 38) (width 0.5) (layer "B.Cu") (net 4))
 (segment (start 32.975 43.19) (end 21.94 43.19) (width 0.5) (layer "B.Cu") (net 4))
 (segment (start 16.75 38) (end 16.75 16.765564) (width 0.5) (layer "B.Cu") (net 4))
 (segment (start 16.75 16.765564) (end 9.25 9.265564) (width 0.5) (layer "B.Cu") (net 4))
 (segment (start 14.75 25.32) (end 11.32 25.32) (width 0.5) (layer "F.Cu") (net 29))
 (segment (start 21.25 25.32) (end 14.75 25.32) (width 0.5) (layer "F.Cu") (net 29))
 (segment (start 14.75 40.25) (end 14.75 25.32) (width 0.5) (layer "B.Cu") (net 29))
 (segment (start 20.23 45.73) (end 14.75 40.25) (width 0.5) (layer "B.Cu") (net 29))
 (segment (start 32.975 45.73) (end 20.23 45.73) (width 0.5) (layer "B.Cu") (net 29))
 (segment (start 28.206 23.005) (end 28.206 23.544) (width 0.5) (layer "F.Cu") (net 33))
 (segment (start 27.6 55.1) (end 28.39 55.89) (width 0.5) (layer "F.Cu") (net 33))
 (segment (start 28.39 55.89) (end 32.975 55.89) (width 0.5) (layer "F.Cu") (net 33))
 (segment (start 27.6 24.15) (end 27.6 55.1) (width 0.5) (layer "F.Cu") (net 33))
 (segment (start 28.206 23.544) (end 27.6 24.15) (width 0.5) (layer "F.Cu") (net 33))
 (segment (start 34.275 57.13) (end 34.275 23.524) (width 0.5) (layer "F.Cu") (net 34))
 (segment (start 32.975 58.43) (end 34.275 57.13) (width 0.5) (layer "F.Cu") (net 34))
 (segment (start 34.275 23.524) (end 31.756 21.005) (width 0.5) (layer "F.Cu") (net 34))
 (segment (start 13.4 78.27) (end 13.4 76.37) (width 0.5) (layer "F.Cu") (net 3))
 (segment (start 8.42 20.82) (end 7.62 21.62) (width 0.5) (layer "F.Cu") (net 3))
 (segment (start 9.25 4.765564) (end 2.75 4.765564) (width 0.5) (layer "F.Cu") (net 3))
 (segment (start 16.25 81.12) (end 14.44 79.31) (width 0.5) (layer "F.Cu") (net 3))
 (segment (start 14.75 20.82) (end 8.42 20.82) (width 0.5) (layer "F.Cu") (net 3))
 (segment (start 12.75 4.765564) (end 9.25 4.765564) (width 0.5) (layer "F.Cu") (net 3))
 (segment (start 14.44 79.31) (end 13.4 78.27) (width 0.5) (layer "F.Cu") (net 3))
 (segment (start 14.75 20.82) (end 21.25 20.82) (width 0.5) (layer "F.Cu") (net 3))
 (segment (start 19.25 4.765564) (end 12.75 4.765564) (width 0.5) (layer "F.Cu") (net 3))
 (via (at 14.44 79.31) (size 0.6) (drill 0.4) (layers "F.Cu" "B.Cu") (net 3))
 (via (at 7.62 21.62) (size 0.6) (drill 0.4) (layers "F.Cu" "B.Cu") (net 3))
 (segment (start 9.2 50.8) (end 10.75 49.25) (width 1) (layer "B.Cu") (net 3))
 (segment (start 10.75 49.25) (end 10.75 37.25) (width 1) (layer "B.Cu") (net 3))
 (segment (start 25.41 68.59) (end 25.16 68.59) (width 0.5) (layer "B.Cu") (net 3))
 (segment (start 6.82 20.82) (end 7.62 21.62) (width 0.5) (layer "B.Cu") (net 3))
 (segment (start 33.505 17.005) (end 31.756 17.005) (width 1) (layer "B.Cu") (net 3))
 (segment (start 9.06 35.56) (end 7.62 35.56) (width 1) (layer "B.Cu") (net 3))
 (segment (start 7.62 50.8) (end 9.2 50.8) (width 1) (layer "B.Cu") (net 3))
 (segment (start 4.2 6.215564) (end 2.75 4.765564) (width 0.5) (layer "B.Cu") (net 3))
 (segment (start 34.525 18.025) (end 33.505 17.005) (width 1) (layer "B.Cu") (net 3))
 (segment (start 10.75 37.25) (end 9.06 35.56) (width 1) (layer "B.Cu") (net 3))
 (segment (start 32.975 68.59) (end 25.41 68.59) (width 1) (layer "B.Cu") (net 3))
 (segment (start 25.16 68.59) (end 14.44 79.31) (width 0.5) (layer "B.Cu") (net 3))
 (segment (start 6.82 20.82) (end 4.2 18.2) (width 0.5) (layer "B.Cu") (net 3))
 (segment (start 34.525 67.04) (end 34.525 18.025) (width 1) (layer "B.Cu") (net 3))
 (segment (start 7.62 50.8) (end 25.41 68.59) (width 1) (layer "B.Cu") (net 3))
 (segment (start 7.62 21.62) (end 7.62 35.56) (width 0.5) (layer "B.Cu") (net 3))
 (segment (start 32.975 68.59) (end 34.525 67.04) (width 1) (layer "B.Cu") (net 3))
 (segment (start 4.2 18.2) (end 4.2 6.215564) (width 0.5) (layer "B.Cu") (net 3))
 (segment (start 30.006 20.005) (end 30.006 15.744) (width 0.5) (layer "F.Cu") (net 38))
 (segment (start 35.675 16.425) (end 35.675 68.43) (width 0.5) (layer "F.Cu") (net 38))
 (segment (start 34.25 15) (end 35.675 16.425) (width 0.5) (layer "F.Cu") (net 38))
 (segment (start 30.006 15.744) (end 30.75 15) (width 0.5) (layer "F.Cu") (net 38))
 (segment (start 35.675 68.43) (end 32.975 71.13) (width 0.5) (layer "F.Cu") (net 38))
 (segment (start 30.75 15) (end 34.25 15) (width 0.5) (layer "F.Cu") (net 38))
 (segment (start 26.2 34.8) (end 26.2 19.55) (width 0.5) (layer "F.Cu") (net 6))
 (segment (start 26.745 19.005) (end 28.256 19.005) (width 0.5) (layer "F.Cu") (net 6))
 (segment (start 26.2 19.55) (end 26.745 19.005) (width 0.5) (layer "F.Cu") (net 6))
 (segment (start 22.9 38.1) (end 26.2 34.8) (width 0.5) (layer "F.Cu") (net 6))
 (segment (start 7.62 38.1) (end 22.9 38.1) (width 0.5) (layer "F.Cu") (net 6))
 (segment (start 9.46 38.8) (end 7.62 40.64) (width 0.5) (layer "F.Cu") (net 7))
 (segment (start 26.9 35.1) (end 23.2 38.8) (width 0.5) (layer "F.Cu") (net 7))
 (segment (start 27.245 21.005) (end 26.9 21.35) (width 0.5) (layer "F.Cu") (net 7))
 (segment (start 28.256 21.005) (end 27.245 21.005) (width 0.5) (layer "F.Cu") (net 7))
 (segment (start 26.9 21.35) (end 26.9 35.1) (width 0.5) (layer "F.Cu") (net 7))
 (segment (start 23.2 38.8) (end 9.46 38.8) (width 0.5) (layer "F.Cu") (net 7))
 (segment (start 3.4 19.08995) (end 3.4 46.4) (width 0.5) (layer "F.Cu") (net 10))
 (segment (start 4.169975 18.319975) (end 3.4 19.08995) (width 0.5) (layer "F.Cu") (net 10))
 (segment (start 3.4 46.4) (end 5.26 48.26) (width 0.5) (layer "F.Cu") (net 10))
 (segment (start 20.5 17) (end 19.180025 18.319975) (width 0.5) (layer "F.Cu") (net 10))
 (segment (start 5.26 48.26) (end 7.62 48.26) (width 0.5) (layer "F.Cu") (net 10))
 (segment (start 19.180025 18.319975) (end 4.169975 18.319975) (width 0.5) (layer "F.Cu") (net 10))
 (via (at 20.5 17) (size 0.6) (drill 0.4) (layers "F.Cu" "B.Cu") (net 10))
 (segment (start 29.23995 7.75) (end 20.5 16.48995) (width 0.5) (layer "B.Cu") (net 10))
 (segment (start 31.7 7.75) (end 29.23995 7.75) (width 0.5) (layer "B.Cu") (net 10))
 (segment (start 34.37 5.08) (end 31.7 7.75) (width 0.5) (layer "B.Cu") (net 10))
 (segment (start 20.5 16.48995) (end 20.5 16.75) (width 0.5) (layer "B.Cu") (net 10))
 (segment (start 20.5 16.75) (end 20.5 17) (width 0.5) (layer "B.Cu") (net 10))
 (segment (start 2.7 51.7) (end 4.34 53.34) (width 0.5) (layer "F.Cu") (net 11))
 (segment (start 2.7 18.8) (end 2.7 51.7) (width 0.5) (layer "F.Cu") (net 11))
 (segment (start 18.130025 17.619975) (end 18.01005 17.5) (width 0.5) (layer "F.Cu") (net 11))
 (segment (start 20.5 15.25) (end 18.130025 17.619975) (width 0.5) (layer "F.Cu") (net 11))
 (segment (start 4 17.5) (end 2.7 18.8) (width 0.5) (layer "F.Cu") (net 11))
 (segment (start 18.01005 17.5) (end 4 17.5) (width 0.5) (layer "F.Cu") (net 11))
 (segment (start 4.34 53.34) (end 7.62 53.34) (width 0.5) (layer "F.Cu") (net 11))
 (via (at 20.5 15.25) (size 0.6) (drill 0.4) (layers "F.Cu" "B.Cu") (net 11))
 (segment (start 28.83 7.17) (end 20.75 15.25) (width 0.5) (layer "B.Cu") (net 11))
 (segment (start 20.75 15.25) (end 20.5 15.25) (width 0.5) (layer "B.Cu") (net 11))
 (segment (start 28.83 5.08) (end 28.83 7.17) (width 0.5) (layer "B.Cu") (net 11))
 (segment (start 3.38 55.88) (end 7.62 55.88) (width 0.5) (layer "F.Cu") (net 12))
 (segment (start 17.51939 16) (end 16.76939 16.75) (width 0.5) (layer "F.Cu") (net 12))
 (segment (start 20.939339 13.75) (end 18.689339 16) (width 0.5) (layer "F.Cu") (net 12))
 (segment (start 16.76939 16.75) (end 3.25 16.75) (width 0.5) (layer "F.Cu") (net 12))
 (segment (start 3.25 16.75) (end 2 18) (width 0.5) (layer "F.Cu") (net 12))
 (segment (start 21 13.75) (end 20.939339 13.75) (width 0.5) (layer "F.Cu") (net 12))
 (segment (start 2 18) (end 2 54.5) (width 0.5) (layer "F.Cu") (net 12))
 (segment (start 2 54.5) (end 3.38 55.88) (width 0.5) (layer "F.Cu") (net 12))
 (segment (start 18.689339 16) (end 17.51939 16) (width 0.5) (layer "F.Cu") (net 12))
 (via (at 21 13.75) (size 0.6) (drill 0.4) (layers "F.Cu" "B.Cu") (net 12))
 (segment (start 23.29 5.08) (end 23.29 11.46) (width 0.5) (layer "B.Cu") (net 12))
 (segment (start 23.29 11.46) (end 21 13.75) (width 0.5) (layer "B.Cu") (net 12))
 (segment (start 15.06 70.31) (end 10.79 66.04) (width 0.5) (layer "F.Cu") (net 16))
 (segment (start 10.79 66.04) (end 7.62 66.04) (width 0.5) (layer "F.Cu") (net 16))
 (segment (start 16.75 71.12) (end 15.06 72.81) (width 0.5) (layer "F.Cu") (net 16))
 (segment (start 15.06 72.81) (end 13.4 74.47) (width 0.5) (layer "F.Cu") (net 16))
 (segment (start 15.06 72.81) (end 15.06 70.31) (width 0.5) (layer "F.Cu") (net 16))
 (segment (start 23.38 75.12) (end 23.38 71.25) (width 0.5) (layer "F.Cu") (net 23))
 (segment (start 23.38 75.12) (end 23.38 75.47) (width 0.5) (layer "F.Cu") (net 23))
 (segment (start 23.38 71.25) (end 23.25 71.12) (width 0.5) (layer "F.Cu") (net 23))
 (segment (start 22.33 76.52) (end 17.5 76.52) (width 0.5) (layer "F.Cu") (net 23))
 (segment (start 23.38 75.47) (end 22.33 76.52) (width 0.5) (layer "F.Cu") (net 23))
 (segment (start 17.5 76.52) (end 16.4 75.42) (width 0.5) (layer "F.Cu") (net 23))
 (segment (start 26 55.25) (end 26 38.75) (width 1) (layer "F.Cu") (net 1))
 (segment (start 28.5 77.5) (end 28.5 57.75) (width 1) (layer "F.Cu") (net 1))
 (segment (start 25.65 80.35) (end 28.5 77.5) (width 1) (layer "F.Cu") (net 1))
 (segment (start 28.5 57.75) (end 26 55.25) (width 1) (layer "F.Cu") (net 1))
 (segment (start 26 38.75) (end 26.5 38.25) (width 1) (layer "F.Cu") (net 1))
 (segment (start 25.65 80.75) (end 25.65 80.35) (width 1) (layer "F.Cu") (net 1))
 (segment (start 26.5 38.25) (end 26.65 38.25) (width 1) (layer "F.Cu") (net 1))
 (via (at 26.75 38.25) (size 0.6) (drill 0.4) (layers "F.Cu" "B.Cu") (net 1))
 (segment (start 25.25 18.25) (end 26.495 17.005) (width 1) (layer "B.Cu") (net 1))
 (segment (start 26.495 17.005) (end 28.256 17.005) (width 1) (layer "B.Cu") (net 1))
 (segment (start 26.75 26.25) (end 25.25 24.75) (width 1) (layer "B.Cu") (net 1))
 (segment (start 26.75 38.25) (end 26.75 26.25) (width 1) (layer "B.Cu") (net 1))
 (segment (start 25.25 24.75) (end 25.25 18.25) (width 1) (layer "B.Cu") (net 1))
 (segment (start 21.25 78.12) (end 18.25 81.12) (width 1) (layer "F.Cu") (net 2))
 (segment (start 23.38 78.12) (end 22.43 78.12) (width 1) (layer "F.Cu") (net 2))
 (segment (start 26.25 72.65) (end 26.25 75.25) (width 1) (layer "F.Cu") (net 2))
 (segment (start 22.43 78.83) (end 24.35 80.75) (width 1) (layer "F.Cu") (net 2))
 (segment (start 22.43 78.12) (end 21.25 78.12) (width 1) (layer "F.Cu") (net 2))
 (segment (start 22.43 78.12) (end 22.43 78.83) (width 1) (layer "F.Cu") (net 2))
 (segment (start 26.25 75.25) (end 23.38 78.12) (width 1) (layer "F.Cu") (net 2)))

